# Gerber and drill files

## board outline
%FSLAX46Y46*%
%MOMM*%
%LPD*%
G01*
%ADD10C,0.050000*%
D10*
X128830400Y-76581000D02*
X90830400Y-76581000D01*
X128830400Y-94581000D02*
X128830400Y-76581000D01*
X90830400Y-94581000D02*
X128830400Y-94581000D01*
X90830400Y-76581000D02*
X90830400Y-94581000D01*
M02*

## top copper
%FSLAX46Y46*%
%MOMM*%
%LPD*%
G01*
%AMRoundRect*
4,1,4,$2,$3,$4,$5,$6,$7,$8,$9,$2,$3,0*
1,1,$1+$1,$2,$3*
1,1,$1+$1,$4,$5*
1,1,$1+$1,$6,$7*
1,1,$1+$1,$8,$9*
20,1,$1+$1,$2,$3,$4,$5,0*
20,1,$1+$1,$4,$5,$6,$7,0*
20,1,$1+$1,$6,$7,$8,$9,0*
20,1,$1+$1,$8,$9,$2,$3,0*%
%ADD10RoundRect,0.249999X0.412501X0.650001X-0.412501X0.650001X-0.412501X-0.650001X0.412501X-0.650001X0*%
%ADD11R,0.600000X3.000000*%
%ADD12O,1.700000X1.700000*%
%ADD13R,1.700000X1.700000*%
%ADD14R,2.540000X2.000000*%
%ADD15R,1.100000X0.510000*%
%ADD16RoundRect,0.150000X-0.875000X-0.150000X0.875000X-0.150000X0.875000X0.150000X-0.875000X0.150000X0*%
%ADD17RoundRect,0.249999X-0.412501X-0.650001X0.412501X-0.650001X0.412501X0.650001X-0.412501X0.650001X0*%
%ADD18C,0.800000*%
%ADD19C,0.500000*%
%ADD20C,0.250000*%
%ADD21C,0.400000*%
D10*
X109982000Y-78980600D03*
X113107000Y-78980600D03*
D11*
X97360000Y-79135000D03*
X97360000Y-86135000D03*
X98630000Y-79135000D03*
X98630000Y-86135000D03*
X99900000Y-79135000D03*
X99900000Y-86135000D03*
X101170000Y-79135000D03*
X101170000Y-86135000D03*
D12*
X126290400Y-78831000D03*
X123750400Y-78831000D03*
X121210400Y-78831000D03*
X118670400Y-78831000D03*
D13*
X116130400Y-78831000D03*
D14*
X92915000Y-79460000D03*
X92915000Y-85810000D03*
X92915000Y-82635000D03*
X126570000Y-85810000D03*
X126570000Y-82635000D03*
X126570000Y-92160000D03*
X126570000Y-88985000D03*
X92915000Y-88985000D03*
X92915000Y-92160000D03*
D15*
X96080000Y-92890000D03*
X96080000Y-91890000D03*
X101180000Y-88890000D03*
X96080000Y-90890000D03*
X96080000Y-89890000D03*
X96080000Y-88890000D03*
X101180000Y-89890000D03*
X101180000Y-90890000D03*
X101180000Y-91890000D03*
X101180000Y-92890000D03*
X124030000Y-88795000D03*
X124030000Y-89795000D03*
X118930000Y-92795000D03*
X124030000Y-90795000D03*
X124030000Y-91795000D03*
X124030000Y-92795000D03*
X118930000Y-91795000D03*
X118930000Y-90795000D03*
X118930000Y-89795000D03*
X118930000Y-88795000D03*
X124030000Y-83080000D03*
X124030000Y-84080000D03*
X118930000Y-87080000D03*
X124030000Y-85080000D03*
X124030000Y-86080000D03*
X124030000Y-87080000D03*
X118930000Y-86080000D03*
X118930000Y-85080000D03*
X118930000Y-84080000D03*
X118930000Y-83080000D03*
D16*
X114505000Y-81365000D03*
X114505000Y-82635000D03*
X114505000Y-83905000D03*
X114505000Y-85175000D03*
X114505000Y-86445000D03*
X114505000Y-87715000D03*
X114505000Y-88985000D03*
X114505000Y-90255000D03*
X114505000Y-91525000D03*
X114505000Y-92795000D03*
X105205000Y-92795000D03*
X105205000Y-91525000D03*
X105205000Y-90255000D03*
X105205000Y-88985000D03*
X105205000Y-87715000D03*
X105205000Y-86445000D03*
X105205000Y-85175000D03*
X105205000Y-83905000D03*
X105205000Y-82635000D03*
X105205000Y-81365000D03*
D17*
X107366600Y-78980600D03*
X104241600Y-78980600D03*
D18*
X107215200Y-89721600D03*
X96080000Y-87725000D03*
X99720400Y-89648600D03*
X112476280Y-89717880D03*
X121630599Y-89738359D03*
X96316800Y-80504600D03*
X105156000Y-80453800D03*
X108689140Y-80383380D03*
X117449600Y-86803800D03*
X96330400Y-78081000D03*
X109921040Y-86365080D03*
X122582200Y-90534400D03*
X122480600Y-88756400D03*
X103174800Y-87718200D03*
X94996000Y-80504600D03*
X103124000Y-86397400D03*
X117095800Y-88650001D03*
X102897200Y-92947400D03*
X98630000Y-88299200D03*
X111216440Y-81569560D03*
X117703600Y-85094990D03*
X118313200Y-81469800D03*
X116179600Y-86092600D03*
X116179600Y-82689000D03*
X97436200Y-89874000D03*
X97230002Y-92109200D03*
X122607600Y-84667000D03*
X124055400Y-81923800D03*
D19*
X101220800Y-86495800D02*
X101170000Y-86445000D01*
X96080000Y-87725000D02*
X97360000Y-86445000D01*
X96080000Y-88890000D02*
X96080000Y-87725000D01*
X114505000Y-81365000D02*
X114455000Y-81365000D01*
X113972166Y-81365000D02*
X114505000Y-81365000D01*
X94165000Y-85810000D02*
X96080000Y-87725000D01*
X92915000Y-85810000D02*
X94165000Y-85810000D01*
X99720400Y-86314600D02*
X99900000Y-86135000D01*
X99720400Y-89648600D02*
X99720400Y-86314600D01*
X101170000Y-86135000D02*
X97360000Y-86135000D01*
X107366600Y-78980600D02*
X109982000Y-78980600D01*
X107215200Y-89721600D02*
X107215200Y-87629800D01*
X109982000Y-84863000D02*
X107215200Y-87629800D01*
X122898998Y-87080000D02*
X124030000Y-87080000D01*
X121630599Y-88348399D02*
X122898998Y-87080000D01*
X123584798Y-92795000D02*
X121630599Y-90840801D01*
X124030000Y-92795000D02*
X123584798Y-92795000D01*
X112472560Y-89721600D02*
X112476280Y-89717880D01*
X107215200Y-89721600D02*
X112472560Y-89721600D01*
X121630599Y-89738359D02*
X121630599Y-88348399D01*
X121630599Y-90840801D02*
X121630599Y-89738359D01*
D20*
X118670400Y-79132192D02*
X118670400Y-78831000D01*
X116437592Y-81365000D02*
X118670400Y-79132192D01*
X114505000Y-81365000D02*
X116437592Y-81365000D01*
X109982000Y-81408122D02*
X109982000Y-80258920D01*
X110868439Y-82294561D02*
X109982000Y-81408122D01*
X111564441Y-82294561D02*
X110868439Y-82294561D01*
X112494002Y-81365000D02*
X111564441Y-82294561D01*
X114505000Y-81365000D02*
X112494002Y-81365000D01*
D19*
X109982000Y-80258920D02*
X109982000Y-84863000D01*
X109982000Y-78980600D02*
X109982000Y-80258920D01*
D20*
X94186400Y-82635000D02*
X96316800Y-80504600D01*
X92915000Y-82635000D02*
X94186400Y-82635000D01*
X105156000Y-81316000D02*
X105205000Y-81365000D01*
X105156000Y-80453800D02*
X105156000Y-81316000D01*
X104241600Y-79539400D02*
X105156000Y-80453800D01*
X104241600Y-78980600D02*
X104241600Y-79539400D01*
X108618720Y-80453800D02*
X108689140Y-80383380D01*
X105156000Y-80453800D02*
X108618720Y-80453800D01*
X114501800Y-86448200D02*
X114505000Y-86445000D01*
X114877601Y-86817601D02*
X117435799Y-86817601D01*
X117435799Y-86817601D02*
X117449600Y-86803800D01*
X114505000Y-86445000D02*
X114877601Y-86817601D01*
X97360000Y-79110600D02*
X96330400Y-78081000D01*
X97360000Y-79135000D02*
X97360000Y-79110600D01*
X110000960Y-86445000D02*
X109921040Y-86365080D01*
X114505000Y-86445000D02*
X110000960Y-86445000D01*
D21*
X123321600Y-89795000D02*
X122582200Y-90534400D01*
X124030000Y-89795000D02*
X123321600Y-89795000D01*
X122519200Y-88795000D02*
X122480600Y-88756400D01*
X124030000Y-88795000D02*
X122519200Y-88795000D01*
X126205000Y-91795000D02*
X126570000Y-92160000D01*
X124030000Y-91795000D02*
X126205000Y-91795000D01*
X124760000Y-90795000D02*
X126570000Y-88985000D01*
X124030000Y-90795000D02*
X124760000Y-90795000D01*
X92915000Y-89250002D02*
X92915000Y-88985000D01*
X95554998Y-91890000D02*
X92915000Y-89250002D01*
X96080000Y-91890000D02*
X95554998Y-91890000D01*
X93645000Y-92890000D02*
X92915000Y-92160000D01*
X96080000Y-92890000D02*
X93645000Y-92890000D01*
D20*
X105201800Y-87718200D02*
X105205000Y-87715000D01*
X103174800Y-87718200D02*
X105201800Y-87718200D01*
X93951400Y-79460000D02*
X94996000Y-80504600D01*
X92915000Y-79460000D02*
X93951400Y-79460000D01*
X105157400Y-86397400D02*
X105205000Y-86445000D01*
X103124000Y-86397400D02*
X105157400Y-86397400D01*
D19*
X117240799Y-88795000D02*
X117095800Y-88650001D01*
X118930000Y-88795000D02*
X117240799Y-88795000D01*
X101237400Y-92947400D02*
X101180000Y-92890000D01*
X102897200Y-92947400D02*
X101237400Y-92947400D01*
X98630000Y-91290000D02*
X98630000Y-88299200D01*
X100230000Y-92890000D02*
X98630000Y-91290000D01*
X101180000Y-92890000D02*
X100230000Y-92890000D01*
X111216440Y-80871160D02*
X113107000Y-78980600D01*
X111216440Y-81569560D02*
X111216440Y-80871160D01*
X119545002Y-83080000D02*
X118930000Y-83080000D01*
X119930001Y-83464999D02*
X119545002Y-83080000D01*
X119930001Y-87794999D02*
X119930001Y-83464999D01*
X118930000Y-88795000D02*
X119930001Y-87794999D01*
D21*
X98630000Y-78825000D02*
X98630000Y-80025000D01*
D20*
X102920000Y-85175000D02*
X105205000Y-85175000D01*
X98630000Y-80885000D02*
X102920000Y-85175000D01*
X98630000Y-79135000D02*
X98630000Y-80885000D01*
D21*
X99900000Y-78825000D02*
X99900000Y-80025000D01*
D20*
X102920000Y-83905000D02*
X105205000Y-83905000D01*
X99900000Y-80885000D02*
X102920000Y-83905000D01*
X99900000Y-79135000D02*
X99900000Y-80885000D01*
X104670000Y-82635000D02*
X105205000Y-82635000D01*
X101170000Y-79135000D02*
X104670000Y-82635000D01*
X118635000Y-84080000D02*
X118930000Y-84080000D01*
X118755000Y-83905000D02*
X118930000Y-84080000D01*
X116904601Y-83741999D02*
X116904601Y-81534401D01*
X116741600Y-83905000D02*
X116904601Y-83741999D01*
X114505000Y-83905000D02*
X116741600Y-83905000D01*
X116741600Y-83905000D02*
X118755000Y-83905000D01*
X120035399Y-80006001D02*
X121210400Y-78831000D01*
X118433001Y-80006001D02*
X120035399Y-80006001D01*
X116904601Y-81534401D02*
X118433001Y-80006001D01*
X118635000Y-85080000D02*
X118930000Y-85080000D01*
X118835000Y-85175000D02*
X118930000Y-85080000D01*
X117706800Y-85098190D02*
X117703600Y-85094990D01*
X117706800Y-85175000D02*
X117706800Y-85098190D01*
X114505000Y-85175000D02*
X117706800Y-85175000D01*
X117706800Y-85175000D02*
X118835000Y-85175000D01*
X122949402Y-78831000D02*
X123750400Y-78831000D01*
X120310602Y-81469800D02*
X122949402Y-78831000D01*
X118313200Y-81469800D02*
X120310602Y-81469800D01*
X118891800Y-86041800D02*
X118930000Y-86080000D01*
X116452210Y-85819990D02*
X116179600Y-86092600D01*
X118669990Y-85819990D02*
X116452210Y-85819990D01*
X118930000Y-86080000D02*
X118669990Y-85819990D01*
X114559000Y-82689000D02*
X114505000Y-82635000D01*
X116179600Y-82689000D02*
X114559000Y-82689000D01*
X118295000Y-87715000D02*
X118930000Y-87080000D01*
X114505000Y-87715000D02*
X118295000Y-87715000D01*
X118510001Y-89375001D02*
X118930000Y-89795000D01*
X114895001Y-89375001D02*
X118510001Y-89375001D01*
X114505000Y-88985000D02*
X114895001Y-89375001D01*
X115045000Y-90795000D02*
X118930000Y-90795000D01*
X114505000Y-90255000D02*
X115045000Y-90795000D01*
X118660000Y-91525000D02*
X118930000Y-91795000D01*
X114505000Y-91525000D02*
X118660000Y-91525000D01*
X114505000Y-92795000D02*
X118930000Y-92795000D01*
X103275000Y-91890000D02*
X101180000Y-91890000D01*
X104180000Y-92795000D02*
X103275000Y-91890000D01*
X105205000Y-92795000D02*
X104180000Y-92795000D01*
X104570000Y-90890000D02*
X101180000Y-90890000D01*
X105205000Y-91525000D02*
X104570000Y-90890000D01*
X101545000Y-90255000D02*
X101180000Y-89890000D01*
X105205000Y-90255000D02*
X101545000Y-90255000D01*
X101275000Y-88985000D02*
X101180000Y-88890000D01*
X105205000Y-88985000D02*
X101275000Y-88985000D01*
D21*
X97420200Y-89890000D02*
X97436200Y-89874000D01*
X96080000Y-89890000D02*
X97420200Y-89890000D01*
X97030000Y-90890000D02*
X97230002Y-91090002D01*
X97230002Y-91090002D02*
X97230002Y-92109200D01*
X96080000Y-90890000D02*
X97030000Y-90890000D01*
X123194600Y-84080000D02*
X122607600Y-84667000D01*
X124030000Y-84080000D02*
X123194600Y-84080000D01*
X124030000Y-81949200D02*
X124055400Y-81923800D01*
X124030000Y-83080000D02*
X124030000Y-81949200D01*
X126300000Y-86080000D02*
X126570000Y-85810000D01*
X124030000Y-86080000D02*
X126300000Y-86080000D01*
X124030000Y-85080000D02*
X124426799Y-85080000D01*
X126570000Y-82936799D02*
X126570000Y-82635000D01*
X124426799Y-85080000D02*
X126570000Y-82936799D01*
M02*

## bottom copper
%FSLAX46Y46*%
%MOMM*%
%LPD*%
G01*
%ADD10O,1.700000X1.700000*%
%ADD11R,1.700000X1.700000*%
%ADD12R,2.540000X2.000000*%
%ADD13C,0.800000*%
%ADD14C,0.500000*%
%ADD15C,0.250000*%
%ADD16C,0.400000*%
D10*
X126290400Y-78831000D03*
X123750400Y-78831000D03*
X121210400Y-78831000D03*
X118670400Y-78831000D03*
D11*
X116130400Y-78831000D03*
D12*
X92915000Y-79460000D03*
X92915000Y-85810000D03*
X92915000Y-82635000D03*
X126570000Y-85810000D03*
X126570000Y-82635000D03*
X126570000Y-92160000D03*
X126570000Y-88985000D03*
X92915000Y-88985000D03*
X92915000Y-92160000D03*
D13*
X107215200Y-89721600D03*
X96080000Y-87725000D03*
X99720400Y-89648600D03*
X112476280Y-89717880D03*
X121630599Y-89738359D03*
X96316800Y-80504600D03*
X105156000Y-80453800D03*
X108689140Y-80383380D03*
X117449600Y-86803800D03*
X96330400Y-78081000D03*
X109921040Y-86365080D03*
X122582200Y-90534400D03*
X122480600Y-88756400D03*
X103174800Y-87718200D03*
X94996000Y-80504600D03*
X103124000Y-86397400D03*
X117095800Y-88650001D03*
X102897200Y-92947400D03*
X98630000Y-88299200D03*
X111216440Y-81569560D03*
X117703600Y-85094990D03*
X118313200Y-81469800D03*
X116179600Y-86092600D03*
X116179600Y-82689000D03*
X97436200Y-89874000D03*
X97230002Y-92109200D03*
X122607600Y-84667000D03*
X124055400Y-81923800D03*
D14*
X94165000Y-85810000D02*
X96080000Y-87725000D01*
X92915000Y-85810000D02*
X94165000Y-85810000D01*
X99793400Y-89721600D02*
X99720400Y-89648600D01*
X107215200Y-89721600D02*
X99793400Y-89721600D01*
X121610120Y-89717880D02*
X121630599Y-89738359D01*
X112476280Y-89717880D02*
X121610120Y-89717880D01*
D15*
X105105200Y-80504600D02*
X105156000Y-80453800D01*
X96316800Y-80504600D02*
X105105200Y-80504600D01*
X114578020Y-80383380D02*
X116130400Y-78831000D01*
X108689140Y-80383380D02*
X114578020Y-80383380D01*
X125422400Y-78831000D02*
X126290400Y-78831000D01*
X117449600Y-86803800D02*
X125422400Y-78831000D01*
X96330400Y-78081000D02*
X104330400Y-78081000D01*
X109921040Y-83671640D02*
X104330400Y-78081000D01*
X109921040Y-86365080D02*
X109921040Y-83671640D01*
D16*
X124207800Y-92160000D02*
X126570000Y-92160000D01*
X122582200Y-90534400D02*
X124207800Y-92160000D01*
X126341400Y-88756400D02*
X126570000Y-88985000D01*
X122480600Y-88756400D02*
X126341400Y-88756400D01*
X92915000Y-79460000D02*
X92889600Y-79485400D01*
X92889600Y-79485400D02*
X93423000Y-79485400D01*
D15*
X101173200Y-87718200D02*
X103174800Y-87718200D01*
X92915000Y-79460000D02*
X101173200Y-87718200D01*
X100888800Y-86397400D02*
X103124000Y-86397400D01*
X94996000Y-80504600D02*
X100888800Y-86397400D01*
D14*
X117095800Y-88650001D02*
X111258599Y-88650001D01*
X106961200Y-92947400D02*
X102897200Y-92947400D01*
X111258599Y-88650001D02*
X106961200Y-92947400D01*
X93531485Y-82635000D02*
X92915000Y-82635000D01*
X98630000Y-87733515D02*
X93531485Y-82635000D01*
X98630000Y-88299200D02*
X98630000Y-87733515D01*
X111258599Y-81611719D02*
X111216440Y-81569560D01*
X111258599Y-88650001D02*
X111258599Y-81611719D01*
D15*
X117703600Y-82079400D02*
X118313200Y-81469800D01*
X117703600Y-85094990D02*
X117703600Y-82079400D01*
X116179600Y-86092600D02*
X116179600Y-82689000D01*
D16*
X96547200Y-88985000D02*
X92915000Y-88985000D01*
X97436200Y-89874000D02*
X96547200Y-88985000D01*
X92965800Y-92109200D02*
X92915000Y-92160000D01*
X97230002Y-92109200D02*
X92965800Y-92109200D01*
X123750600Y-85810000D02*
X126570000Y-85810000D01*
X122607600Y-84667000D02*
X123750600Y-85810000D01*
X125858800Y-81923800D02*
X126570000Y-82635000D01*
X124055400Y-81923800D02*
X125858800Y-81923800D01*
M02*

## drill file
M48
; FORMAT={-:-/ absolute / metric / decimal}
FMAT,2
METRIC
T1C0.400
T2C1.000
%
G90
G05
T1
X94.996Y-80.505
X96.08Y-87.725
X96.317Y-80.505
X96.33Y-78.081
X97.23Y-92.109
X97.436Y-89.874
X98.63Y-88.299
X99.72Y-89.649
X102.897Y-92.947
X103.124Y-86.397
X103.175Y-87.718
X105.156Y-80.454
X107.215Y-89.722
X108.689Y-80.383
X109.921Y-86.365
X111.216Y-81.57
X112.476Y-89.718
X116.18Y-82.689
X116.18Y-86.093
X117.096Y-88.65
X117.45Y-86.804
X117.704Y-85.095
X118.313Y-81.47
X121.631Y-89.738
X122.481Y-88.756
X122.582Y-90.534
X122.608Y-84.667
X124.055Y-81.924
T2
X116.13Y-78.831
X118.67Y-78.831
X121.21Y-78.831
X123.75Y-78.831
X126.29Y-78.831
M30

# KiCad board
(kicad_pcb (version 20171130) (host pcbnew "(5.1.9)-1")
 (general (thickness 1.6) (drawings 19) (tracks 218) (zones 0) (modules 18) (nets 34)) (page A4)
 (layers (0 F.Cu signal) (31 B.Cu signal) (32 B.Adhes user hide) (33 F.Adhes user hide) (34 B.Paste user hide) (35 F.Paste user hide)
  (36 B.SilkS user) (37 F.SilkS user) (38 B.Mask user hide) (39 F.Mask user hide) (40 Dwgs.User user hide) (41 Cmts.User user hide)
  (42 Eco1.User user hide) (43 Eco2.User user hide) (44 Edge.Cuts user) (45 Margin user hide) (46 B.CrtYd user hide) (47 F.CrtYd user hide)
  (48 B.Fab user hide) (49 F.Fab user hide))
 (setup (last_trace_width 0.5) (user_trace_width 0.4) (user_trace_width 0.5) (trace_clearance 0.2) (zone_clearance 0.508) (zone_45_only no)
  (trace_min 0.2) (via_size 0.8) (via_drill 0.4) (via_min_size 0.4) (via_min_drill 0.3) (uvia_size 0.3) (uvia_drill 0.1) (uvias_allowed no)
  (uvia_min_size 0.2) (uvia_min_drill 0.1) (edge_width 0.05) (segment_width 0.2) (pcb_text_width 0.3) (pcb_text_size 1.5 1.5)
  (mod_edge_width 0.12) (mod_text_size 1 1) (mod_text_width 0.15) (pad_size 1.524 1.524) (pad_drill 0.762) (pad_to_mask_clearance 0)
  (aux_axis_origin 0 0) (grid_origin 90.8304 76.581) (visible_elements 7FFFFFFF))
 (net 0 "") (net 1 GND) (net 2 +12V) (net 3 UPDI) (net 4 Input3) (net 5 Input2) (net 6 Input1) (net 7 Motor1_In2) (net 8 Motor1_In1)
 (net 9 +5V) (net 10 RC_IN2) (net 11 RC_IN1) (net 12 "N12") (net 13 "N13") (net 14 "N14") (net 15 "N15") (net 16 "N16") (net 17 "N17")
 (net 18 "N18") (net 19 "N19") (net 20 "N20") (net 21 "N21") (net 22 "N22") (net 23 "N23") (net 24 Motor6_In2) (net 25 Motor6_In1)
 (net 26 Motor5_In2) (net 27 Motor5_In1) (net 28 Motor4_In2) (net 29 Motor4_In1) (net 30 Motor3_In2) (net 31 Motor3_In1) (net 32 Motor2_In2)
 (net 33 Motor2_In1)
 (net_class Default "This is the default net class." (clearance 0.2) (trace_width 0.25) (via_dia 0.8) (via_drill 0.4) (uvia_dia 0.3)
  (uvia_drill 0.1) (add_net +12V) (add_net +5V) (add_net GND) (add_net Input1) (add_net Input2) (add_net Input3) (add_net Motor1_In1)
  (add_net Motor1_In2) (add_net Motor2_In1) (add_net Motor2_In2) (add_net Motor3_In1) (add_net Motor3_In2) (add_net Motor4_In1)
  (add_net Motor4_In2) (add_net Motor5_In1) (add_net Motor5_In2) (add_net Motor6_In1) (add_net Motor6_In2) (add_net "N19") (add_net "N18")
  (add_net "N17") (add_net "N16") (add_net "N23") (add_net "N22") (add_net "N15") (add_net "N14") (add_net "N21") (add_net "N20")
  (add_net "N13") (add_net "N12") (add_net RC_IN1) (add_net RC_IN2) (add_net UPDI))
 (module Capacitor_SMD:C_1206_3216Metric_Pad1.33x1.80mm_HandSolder (layer F.Cu) (at 111.5445 78.9806 180)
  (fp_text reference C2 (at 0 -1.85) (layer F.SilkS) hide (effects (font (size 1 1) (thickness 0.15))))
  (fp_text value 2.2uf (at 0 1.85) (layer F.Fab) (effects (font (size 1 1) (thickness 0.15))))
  (pad 2 smd roundrect (at 1.5625 0 180) (size 1.325 1.8) (layers F.Cu F.Paste F.Mask) (roundrect_rratio 0.1886784905660377) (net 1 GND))
  (pad 1 smd roundrect (at -1.5625 0 180) (size 1.325 1.8) (layers F.Cu F.Paste F.Mask) (roundrect_rratio 0.1886784905660377) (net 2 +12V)))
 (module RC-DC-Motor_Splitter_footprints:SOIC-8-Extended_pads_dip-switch (layer F.Cu) (at 99.265 82.635 180)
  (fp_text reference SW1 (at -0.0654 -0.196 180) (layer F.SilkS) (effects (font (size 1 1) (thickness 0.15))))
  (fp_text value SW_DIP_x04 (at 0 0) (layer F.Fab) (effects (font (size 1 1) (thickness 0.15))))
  (pad 4 smd rect (at 1.905 3.5 180) (size 0.6 3) (layers F.Cu F.Paste F.Mask) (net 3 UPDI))
  (pad 5 smd rect (at 1.905 -3.5 180) (size 0.6 3) (layers F.Cu F.Paste F.Mask) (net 1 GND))
  (pad 3 smd rect (at 0.635 3.5 180) (size 0.6 3) (layers F.Cu F.Paste F.Mask) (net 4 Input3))
  (pad 6 smd rect (at 0.635 -3.5 180) (size 0.6 3) (layers F.Cu F.Paste F.Mask) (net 1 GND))
  (pad 2 smd rect (at -0.635 3.5 180) (size 0.6 3) (layers F.Cu F.Paste F.Mask) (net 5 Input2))
  (pad 7 smd rect (at -0.635 -3.5 180) (size 0.6 3) (layers F.Cu F.Paste F.Mask) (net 1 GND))
  (pad 1 smd rect (at -1.905 3.5 180) (size 0.6 3) (layers F.Cu F.Paste F.Mask) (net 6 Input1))
  (pad 8 smd rect (at -1.905 -3.5 180) (size 0.6 3) (layers F.Cu F.Paste F.Mask) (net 1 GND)))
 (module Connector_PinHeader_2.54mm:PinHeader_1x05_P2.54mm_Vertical (layer F.Cu) (at 116.1304 78.831 90)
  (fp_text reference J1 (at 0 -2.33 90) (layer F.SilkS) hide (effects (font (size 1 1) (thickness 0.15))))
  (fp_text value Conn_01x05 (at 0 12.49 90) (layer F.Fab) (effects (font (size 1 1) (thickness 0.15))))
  (pad 5 thru_hole oval (at 0 10.16 90) (size 1.7 1.7) (drill 1) (layers *.Cu *.Mask) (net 3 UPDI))
  (pad 4 thru_hole oval (at 0 7.62 90) (size 1.7 1.7) (drill 1) (layers *.Cu *.Mask) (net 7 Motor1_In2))
  (pad 3 thru_hole oval (at 0 5.08 90) (size 1.7 1.7) (drill 1) (layers *.Cu *.Mask) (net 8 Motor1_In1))
  (pad 2 thru_hole oval (at 0 2.54 90) (size 1.7 1.7) (drill 1) (layers *.Cu *.Mask) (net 1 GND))
  (pad 1 thru_hole rect (at 0 0 90) (size 1.7 1.7) (drill 1) (layers *.Cu *.Mask) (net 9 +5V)))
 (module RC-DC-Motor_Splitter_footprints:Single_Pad (layer F.Cu) (at 92.915 79.46 90)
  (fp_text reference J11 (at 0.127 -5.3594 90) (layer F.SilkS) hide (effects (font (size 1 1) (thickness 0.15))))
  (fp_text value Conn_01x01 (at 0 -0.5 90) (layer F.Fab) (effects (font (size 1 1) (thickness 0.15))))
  (pad 1 smd rect (at 0 0 90) (size 2 2.54) (layers F.Cu F.Paste F.Mask) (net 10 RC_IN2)))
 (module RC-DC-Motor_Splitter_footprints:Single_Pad (layer B.Cu) (at 92.915 79.46 270)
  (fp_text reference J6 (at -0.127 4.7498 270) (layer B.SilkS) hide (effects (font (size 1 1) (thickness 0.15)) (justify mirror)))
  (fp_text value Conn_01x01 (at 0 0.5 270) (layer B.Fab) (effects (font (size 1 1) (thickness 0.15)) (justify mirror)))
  (pad 1 smd rect (at 0 0 270) (size 2 2.54) (layers B.Cu B.Paste B.Mask) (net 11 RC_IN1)))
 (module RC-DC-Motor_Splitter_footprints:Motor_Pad (layer F.Cu) (at 92.915 82.635 270)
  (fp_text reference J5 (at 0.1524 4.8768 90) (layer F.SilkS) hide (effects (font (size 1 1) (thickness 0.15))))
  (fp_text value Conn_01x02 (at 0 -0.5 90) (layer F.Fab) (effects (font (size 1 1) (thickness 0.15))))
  (pad 2 smd rect (at 3.175 0 270) (size 2 2.54) (layers F.Cu F.Paste F.Mask) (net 1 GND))
  (pad 1 smd rect (at 0 0 270) (size 2 2.54) (layers F.Cu F.Paste F.Mask) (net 9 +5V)))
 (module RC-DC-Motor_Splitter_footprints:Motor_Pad (layer B.Cu) (at 92.915 82.635 270)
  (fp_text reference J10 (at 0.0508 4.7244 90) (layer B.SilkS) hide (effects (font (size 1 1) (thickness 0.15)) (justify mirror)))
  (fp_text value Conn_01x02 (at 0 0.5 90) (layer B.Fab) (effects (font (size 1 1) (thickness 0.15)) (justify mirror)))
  (pad 2 smd rect (at 3.175 0 270) (size 2 2.54) (layers B.Cu B.Paste B.Mask) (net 1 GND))
  (pad 1 smd rect (at 0 0 270) (size 2 2.54) (layers B.Cu B.Paste B.Mask) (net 2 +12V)))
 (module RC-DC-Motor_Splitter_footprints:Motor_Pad (layer F.Cu) (at 126.57 82.635 270)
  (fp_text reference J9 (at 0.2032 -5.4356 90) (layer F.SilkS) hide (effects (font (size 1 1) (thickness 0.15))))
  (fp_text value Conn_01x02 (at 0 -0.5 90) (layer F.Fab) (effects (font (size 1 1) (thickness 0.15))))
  (pad 2 smd rect (at 3.175 0 270) (size 2 2.54) (layers F.Cu F.Paste F.Mask) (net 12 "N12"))
  (pad 1 smd rect (at 0 0 270) (size 2 2.54) (layers F.Cu F.Paste F.Mask) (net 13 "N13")))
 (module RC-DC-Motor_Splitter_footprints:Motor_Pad (layer B.Cu) (at 126.57 82.635 270)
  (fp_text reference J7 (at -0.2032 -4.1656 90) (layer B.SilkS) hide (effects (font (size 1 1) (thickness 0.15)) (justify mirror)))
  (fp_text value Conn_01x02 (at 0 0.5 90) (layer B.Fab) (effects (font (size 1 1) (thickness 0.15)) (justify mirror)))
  (pad 2 smd rect (at 3.175 0 270) (size 2 2.54) (layers B.Cu B.Paste B.Mask) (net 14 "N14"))
  (pad 1 smd rect (at 0 0 270) (size 2 2.54) (layers B.Cu B.Paste B.Mask) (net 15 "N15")))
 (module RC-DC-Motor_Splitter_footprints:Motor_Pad (layer F.Cu) (at 126.57 88.985 270)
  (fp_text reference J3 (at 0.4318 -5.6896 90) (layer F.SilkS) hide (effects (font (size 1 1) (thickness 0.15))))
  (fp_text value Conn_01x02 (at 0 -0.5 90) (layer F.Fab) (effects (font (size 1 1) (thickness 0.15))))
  (pad 2 smd rect (at 3.175 0 270) (size 2 2.54) (layers F.Cu F.Paste F.Mask) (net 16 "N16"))
  (pad 1 smd rect (at 0 0 270) (size 2 2.54) (layers F.Cu F.Paste F.Mask) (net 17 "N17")))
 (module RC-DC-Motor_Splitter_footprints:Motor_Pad (layer B.Cu) (at 126.57 88.985 270)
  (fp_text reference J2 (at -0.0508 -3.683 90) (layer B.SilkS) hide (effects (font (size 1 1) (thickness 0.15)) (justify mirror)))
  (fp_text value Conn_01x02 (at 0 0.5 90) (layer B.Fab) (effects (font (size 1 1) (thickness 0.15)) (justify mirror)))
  (pad 2 smd rect (at 3.175 0 270) (size 2 2.54) (layers B.Cu B.Paste B.Mask) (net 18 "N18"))
  (pad 1 smd rect (at 0 0 270) (size 2 2.54) (layers B.Cu B.Paste B.Mask) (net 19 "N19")))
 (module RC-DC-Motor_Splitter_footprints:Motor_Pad (layer B.Cu) (at 92.915 92.16 90)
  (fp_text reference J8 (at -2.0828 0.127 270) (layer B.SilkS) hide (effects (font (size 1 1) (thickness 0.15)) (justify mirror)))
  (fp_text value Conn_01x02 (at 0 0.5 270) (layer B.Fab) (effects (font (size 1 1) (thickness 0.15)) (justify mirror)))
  (pad 2 smd rect (at 3.175 0 90) (size 2 2.54) (layers B.Cu B.Paste B.Mask) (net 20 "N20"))
  (pad 1 smd rect (at 0 0 90) (size 2 2.54) (layers B.Cu B.Paste B.Mask) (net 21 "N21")))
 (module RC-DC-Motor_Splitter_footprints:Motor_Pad (layer F.Cu) (at 92.915 92.16 90)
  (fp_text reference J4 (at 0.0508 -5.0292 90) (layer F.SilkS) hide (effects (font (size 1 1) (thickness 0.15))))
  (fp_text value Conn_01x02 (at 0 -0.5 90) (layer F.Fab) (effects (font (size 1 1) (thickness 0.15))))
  (pad 2 smd rect (at 3.175 0 90) (size 2 2.54) (layers F.Cu F.Paste F.Mask) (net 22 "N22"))
  (pad 1 smd rect (at 0 0 90) (size 2 2.54) (layers F.Cu F.Paste F.Mask) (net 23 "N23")))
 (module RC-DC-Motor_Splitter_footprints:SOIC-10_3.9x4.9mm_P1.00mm (layer F.Cu) (at 98.63 90.89 180)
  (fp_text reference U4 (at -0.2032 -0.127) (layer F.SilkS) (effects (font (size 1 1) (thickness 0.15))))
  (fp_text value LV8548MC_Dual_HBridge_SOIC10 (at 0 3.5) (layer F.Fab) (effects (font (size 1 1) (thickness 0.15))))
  (pad 10 smd rect (at 2.55 -2 180) (size 1.1 0.51) (layers F.Cu F.Paste F.Mask) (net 23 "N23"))
  (pad 9 smd rect (at 2.55 -1 180) (size 1.1 0.51) (layers F.Cu F.Paste F.Mask) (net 22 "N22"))
  (pad 5 smd rect (at -2.55 2 180) (size 1.1 0.51) (layers F.Cu F.Paste F.Mask) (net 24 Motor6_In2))
  (pad 8 smd rect (at 2.55 0 180) (size 1.1 0.51) (layers F.Cu F.Paste F.Mask) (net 21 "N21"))
  (pad 7 smd rect (at 2.55 1 180) (size 1.1 0.51) (layers F.Cu F.Paste F.Mask) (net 20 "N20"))
  (pad 6 smd rect (at 2.55 2 180) (size 1.1 0.51) (layers F.Cu F.Paste F.Mask) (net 1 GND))
  (pad 4 smd rect (at -2.55 1 180) (size 1.1 0.51) (layers F.Cu F.Paste F.Mask) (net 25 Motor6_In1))
  (pad 3 smd rect (at -2.55 0 180) (size 1.1 0.51) (layers F.Cu F.Paste F.Mask) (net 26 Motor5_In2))
  (pad 2 smd rect (at -2.55 -1 180) (size 1.1 0.51) (layers F.Cu F.Paste F.Mask) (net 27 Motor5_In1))
  (pad 1 smd rect (at -2.55 -2 180) (size 1.1 0.51) (layers F.Cu F.Paste F.Mask) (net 2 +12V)))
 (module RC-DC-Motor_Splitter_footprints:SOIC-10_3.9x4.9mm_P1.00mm (layer F.Cu) (at 121.48 90.795)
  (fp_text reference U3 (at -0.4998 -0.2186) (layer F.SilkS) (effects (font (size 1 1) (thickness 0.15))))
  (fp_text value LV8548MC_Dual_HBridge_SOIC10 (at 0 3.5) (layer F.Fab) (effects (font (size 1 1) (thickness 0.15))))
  (pad 10 smd rect (at 2.55 -2) (size 1.1 0.51) (layers F.Cu F.Paste F.Mask) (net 19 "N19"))
  (pad 9 smd rect (at 2.55 -1) (size 1.1 0.51) (layers F.Cu F.Paste F.Mask) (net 18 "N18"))
  (pad 5 smd rect (at -2.55 2) (size 1.1 0.51) (layers F.Cu F.Paste F.Mask) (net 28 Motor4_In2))
  (pad 8 smd rect (at 2.55 0) (size 1.1 0.51) (layers F.Cu F.Paste F.Mask) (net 17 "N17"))
  (pad 7 smd rect (at 2.55 1) (size 1.1 0.51) (layers F.Cu F.Paste F.Mask) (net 16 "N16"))
  (pad 6 smd rect (at 2.55 2) (size 1.1 0.51) (layers F.Cu F.Paste F.Mask) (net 1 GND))
  (pad 4 smd rect (at -2.55 1) (size 1.1 0.51) (layers F.Cu F.Paste F.Mask) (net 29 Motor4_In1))
  (pad 3 smd rect (at -2.55 0) (size 1.1 0.51) (layers F.Cu F.Paste F.Mask) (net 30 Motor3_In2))
  (pad 2 smd rect (at -2.55 -1) (size 1.1 0.51) (layers F.Cu F.Paste F.Mask) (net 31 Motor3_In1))
  (pad 1 smd rect (at -2.55 -2) (size 1.1 0.51) (layers F.Cu F.Paste F.Mask) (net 2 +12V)))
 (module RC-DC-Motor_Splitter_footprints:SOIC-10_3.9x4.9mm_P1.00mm (layer F.Cu) (at 121.48 85.08)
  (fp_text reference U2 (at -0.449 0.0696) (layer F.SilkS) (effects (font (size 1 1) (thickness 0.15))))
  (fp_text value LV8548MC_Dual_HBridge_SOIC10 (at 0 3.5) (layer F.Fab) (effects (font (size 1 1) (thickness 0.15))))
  (pad 10 smd rect (at 2.55 -2) (size 1.1 0.51) (layers F.Cu F.Paste F.Mask) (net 15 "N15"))
  (pad 9 smd rect (at 2.55 -1) (size 1.1 0.51) (layers F.Cu F.Paste F.Mask) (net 14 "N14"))
  (pad 5 smd rect (at -2.55 2) (size 1.1 0.51) (layers F.Cu F.Paste F.Mask) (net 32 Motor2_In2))
  (pad 8 smd rect (at 2.55 0) (size 1.1 0.51) (layers F.Cu F.Paste F.Mask) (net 13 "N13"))
  (pad 7 smd rect (at 2.55 1) (size 1.1 0.51) (layers F.Cu F.Paste F.Mask) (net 12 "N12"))
  (pad 6 smd rect (at 2.55 2) (size 1.1 0.51) (layers F.Cu F.Paste F.Mask) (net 1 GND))
  (pad 4 smd rect (at -2.55 1) (size 1.1 0.51) (layers F.Cu F.Paste F.Mask) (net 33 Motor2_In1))
  (pad 3 smd rect (at -2.55 0) (size 1.1 0.51) (layers F.Cu F.Paste F.Mask) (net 7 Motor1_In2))
  (pad 2 smd rect (at -2.55 -1) (size 1.1 0.51) (layers F.Cu F.Paste F.Mask) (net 8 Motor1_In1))
  (pad 1 smd rect (at -2.55 -2) (size 1.1 0.51) (layers F.Cu F.Paste F.Mask) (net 2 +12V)))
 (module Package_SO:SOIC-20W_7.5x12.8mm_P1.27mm (layer F.Cu) (at 109.855 87.08)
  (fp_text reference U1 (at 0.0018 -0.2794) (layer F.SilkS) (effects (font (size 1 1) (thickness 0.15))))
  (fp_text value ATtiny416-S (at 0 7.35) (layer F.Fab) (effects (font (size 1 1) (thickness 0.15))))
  (pad 20 smd roundrect (at 4.65 -5.715) (size 2.05 0.6) (layers F.Cu F.Paste F.Mask) (roundrect_rratio 0.25) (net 1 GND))
  (pad 19 smd roundrect (at 4.65 -4.445) (size 2.05 0.6) (layers F.Cu F.Paste F.Mask) (roundrect_rratio 0.25) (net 33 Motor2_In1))
  (pad 18 smd roundrect (at 4.65 -3.175) (size 2.05 0.6) (layers F.Cu F.Paste F.Mask) (roundrect_rratio 0.25) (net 8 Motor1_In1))
  (pad 17 smd roundrect (at 4.65 -1.905) (size 2.05 0.6) (layers F.Cu F.Paste F.Mask) (roundrect_rratio 0.25) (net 7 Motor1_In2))
  (pad 16 smd roundrect (at 4.65 -0.635) (size 2.05 0.6) (layers F.Cu F.Paste F.Mask) (roundrect_rratio 0.25) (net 3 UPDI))
  (pad 15 smd roundrect (at 4.65 0.635) (size 2.05 0.6) (layers F.Cu F.Paste F.Mask) (roundrect_rratio 0.25) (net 32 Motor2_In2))
  (pad 14 smd roundrect (at 4.65 1.905) (size 2.05 0.6) (layers F.Cu F.Paste F.Mask) (roundrect_rratio 0.25) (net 31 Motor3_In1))
  (pad 13 smd roundrect (at 4.65 3.175) (size 2.05 0.6) (layers F.Cu F.Paste F.Mask) (roundrect_rratio 0.25) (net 30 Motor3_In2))
  (pad 12 smd roundrect (at 4.65 4.445) (size 2.05 0.6) (layers F.Cu F.Paste F.Mask) (roundrect_rratio 0.25) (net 29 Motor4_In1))
  (pad 11 smd roundrect (at 4.65 5.715) (size 2.05 0.6) (layers F.Cu F.Paste F.Mask) (roundrect_rratio 0.25) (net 28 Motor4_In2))
  (pad 10 smd roundrect (at -4.65 5.715) (size 2.05 0.6) (layers F.Cu F.Paste F.Mask) (roundrect_rratio 0.25) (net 27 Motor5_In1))
  (pad 9 smd roundrect (at -4.65 4.445) (size 2.05 0.6) (layers F.Cu F.Paste F.Mask) (roundrect_rratio 0.25) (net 26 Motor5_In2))
  (pad 8 smd roundrect (at -4.65 3.175) (size 2.05 0.6) (layers F.Cu F.Paste F.Mask) (roundrect_rratio 0.25) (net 25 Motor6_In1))
  (pad 7 smd roundrect (at -4.65 1.905) (size 2.05 0.6) (layers F.Cu F.Paste F.Mask) (roundrect_rratio 0.25) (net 24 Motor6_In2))
  (pad 6 smd roundrect (at -4.65 0.635) (size 2.05 0.6) (layers F.Cu F.Paste F.Mask) (roundrect_rratio 0.25) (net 11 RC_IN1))
  (pad 5 smd roundrect (at -4.65 -0.635) (size 2.05 0.6) (layers F.Cu F.Paste F.Mask) (roundrect_rratio 0.25) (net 10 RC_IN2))
  (pad 4 smd roundrect (at -4.65 -1.905) (size 2.05 0.6) (layers F.Cu F.Paste F.Mask) (roundrect_rratio 0.25) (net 4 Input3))
  (pad 3 smd roundrect (at -4.65 -3.175) (size 2.05 0.6) (layers F.Cu F.Paste F.Mask) (roundrect_rratio 0.25) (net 5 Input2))
  (pad 2 smd roundrect (at -4.65 -4.445) (size 2.05 0.6) (layers F.Cu F.Paste F.Mask) (roundrect_rratio 0.25) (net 6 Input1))
  (pad 1 smd roundrect (at -4.65 -5.715) (size 2.05 0.6) (layers F.Cu F.Paste F.Mask) (roundrect_rratio 0.25) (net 9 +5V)))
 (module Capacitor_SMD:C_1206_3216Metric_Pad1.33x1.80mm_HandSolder (layer F.Cu) (at 105.8041 78.9806)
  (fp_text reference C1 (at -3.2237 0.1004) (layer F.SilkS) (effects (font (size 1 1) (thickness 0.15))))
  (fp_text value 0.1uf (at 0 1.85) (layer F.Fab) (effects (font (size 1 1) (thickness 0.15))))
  (pad 2 smd roundrect (at 1.5625 0) (size 1.325 1.8) (layers F.Cu F.Paste F.Mask) (roundrect_rratio 0.1886784905660377) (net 1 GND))
  (pad 1 smd roundrect (at -1.5625 0) (size 1.325 1.8) (layers F.Cu F.Paste F.Mask) (roundrect_rratio 0.1886784905660377) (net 9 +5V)))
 (gr_line (start 128.8304 76.581) (end 90.8304 76.581) (layer Edge.Cuts) (width 0.05))
 (gr_line (start 128.8304 94.581) (end 128.8304 76.581) (layer Edge.Cuts) (width 0.05))
 (gr_line (start 90.8304 94.581) (end 128.8304 94.581) (layer Edge.Cuts) (width 0.05))
 (gr_line (start 90.8304 76.581) (end 90.8304 94.581) (layer Edge.Cuts) (width 0.05))
 (via (at 107.2152 89.7216) (size 0.8) (drill 0.4) (layers F.Cu B.Cu) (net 1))
 (segment (start 101.2208 86.4958) (end 101.17 86.445) (width 0.5) (layer F.Cu) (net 1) (status 30))
 (segment (start 96.08 87.725) (end 97.36 86.445) (width 0.5) (layer F.Cu) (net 1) (status 20))
 (segment (start 96.08 88.89) (end 96.08 87.725) (width 0.5) (layer F.Cu) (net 1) (status 10))
 (segment (start 114.505 81.365) (end 114.455 81.365) (width 0.5) (layer F.Cu) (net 1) (status 30))
 (segment (start 113.972166 81.365) (end 114.505 81.365) (width 0.5) (layer F.Cu) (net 1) (status 30))
 (via (at 96.08 87.725) (size 0.8) (drill 0.4) (layers F.Cu B.Cu) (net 1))
 (segment (start 94.165 85.81) (end 96.08 87.725) (width 0.5) (layer B.Cu) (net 1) (status 10))
 (segment (start 92.915 85.81) (end 94.165 85.81) (width 0.5) (layer B.Cu) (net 1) (status 30))
 (segment (start 94.165 85.81) (end 96.08 87.725) (width 0.5) (layer F.Cu) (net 1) (status 10))
 (segment (start 92.915 85.81) (end 94.165 85.81) (width 0.5) (layer F.Cu) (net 1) (status 30))
 (via (at 99.7204 89.6486) (size 0.8) (drill 0.4) (layers F.Cu B.Cu) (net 1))
 (segment (start 99.7934 89.7216) (end 99.7204 89.6486) (width 0.5) (layer B.Cu) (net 1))
 (segment (start 107.2152 89.7216) (end 99.7934 89.7216) (width 0.5) (layer B.Cu) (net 1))
 (segment (start 99.7204 86.3146) (end 99.9 86.135) (width 0.5) (layer F.Cu) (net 1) (status 30))
 (segment (start 99.7204 89.6486) (end 99.7204 86.3146) (width 0.5) (layer F.Cu) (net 1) (status 20))
 (segment (start 101.17 86.135) (end 97.36 86.135) (width 0.5) (layer F.Cu) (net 1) (status 30))
 (segment (start 107.3666 78.9806) (end 109.982 78.9806) (width 0.5) (layer F.Cu) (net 1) (status 30))
 (segment (start 107.2152 89.7216) (end 107.2152 87.6298) (width 0.5) (layer F.Cu) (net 1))
 (segment (start 109.982 84.863) (end 107.2152 87.6298) (width 0.5) (layer F.Cu) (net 1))
 (segment (start 122.898998 87.08) (end 124.03 87.08) (width 0.5) (layer F.Cu) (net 1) (status 20))
 (segment (start 121.630599 88.348399) (end 122.898998 87.08) (width 0.5) (layer F.Cu) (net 1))
 (segment (start 123.584798 92.795) (end 121.630599 90.840801) (width 0.5) (layer F.Cu) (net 1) (status 10))
 (segment (start 124.03 92.795) (end 123.584798 92.795) (width 0.5) (layer F.Cu) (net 1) (status 30))
 (via (at 112.47628 89.71788) (size 0.8) (drill 0.4) (layers F.Cu B.Cu) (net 1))
 (segment (start 112.47256 89.7216) (end 112.47628 89.71788) (width 0.5) (layer F.Cu) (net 1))
 (segment (start 107.2152 89.7216) (end 112.47256 89.7216) (width 0.5) (layer F.Cu) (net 1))
 (via (at 121.630599 89.738359) (size 0.8) (drill 0.4) (layers F.Cu B.Cu) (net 1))
 (segment (start 121.61012 89.71788) (end 121.630599 89.738359) (width 0.5) (layer B.Cu) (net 1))
 (segment (start 112.47628 89.71788) (end 121.61012 89.71788) (width 0.5) (layer B.Cu) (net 1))
 (segment (start 121.630599 89.738359) (end 121.630599 88.348399) (width 0.5) (layer F.Cu) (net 1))
 (segment (start 121.630599 90.840801) (end 121.630599 89.738359) (width 0.5) (layer F.Cu) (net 1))
 (segment (start 118.6704 79.132192) (end 118.6704 78.831) (width 0.25) (layer F.Cu) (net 1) (status 30))
 (segment (start 116.437592 81.365) (end 118.6704 79.132192) (width 0.25) (layer F.Cu) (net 1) (status 20))
 (segment (start 114.505 81.365) (end 116.437592 81.365) (width 0.25) (layer F.Cu) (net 1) (status 10))
 (segment (start 109.982 81.408122) (end 109.982 80.25892) (width 0.25) (layer F.Cu) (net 1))
 (segment (start 110.868439 82.294561) (end 109.982 81.408122) (width 0.25) (layer F.Cu) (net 1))
 (segment (start 111.564441 82.294561) (end 110.868439 82.294561) (width 0.25) (layer F.Cu) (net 1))
 (segment (start 112.494002 81.365) (end 111.564441 82.294561) (width 0.25) (layer F.Cu) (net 1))
 (segment (start 114.505 81.365) (end 112.494002 81.365) (width 0.25) (layer F.Cu) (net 1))
 (segment (start 109.982 80.25892) (end 109.982 84.863) (width 0.5) (layer F.Cu) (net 1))
 (segment (start 109.982 78.9806) (end 109.982 80.25892) (width 0.5) (layer F.Cu) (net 1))
 (via (at 96.3168 80.5046) (size 0.8) (drill 0.4) (layers F.Cu B.Cu) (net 9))
 (segment (start 94.1864 82.635) (end 96.3168 80.5046) (width 0.25) (layer F.Cu) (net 9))
 (segment (start 92.915 82.635) (end 94.1864 82.635) (width 0.25) (layer F.Cu) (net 9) (status 10))
 (via (at 105.156 80.4538) (size 0.8) (drill 0.4) (layers F.Cu B.Cu) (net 9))
 (segment (start 105.1052 80.5046) (end 105.156 80.4538) (width 0.25) (layer B.Cu) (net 9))
 (segment (start 96.3168 80.5046) (end 105.1052 80.5046) (width 0.25) (layer B.Cu) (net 9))
 (segment (start 105.156 81.316) (end 105.205 81.365) (width 0.25) (layer F.Cu) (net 9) (status 30))
 (segment (start 105.156 80.4538) (end 105.156 81.316) (width 0.25) (layer F.Cu) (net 9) (status 20))
 (segment (start 104.2416 79.5394) (end 105.156 80.4538) (width 0.25) (layer F.Cu) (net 9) (status 10))
 (segment (start 104.2416 78.9806) (end 104.2416 79.5394) (width 0.25) (layer F.Cu) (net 9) (status 30))
 (via (at 108.68914 80.38338) (size 0.8) (drill 0.4) (layers F.Cu B.Cu) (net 9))
 (segment (start 108.61872 80.4538) (end 108.68914 80.38338) (width 0.25) (layer F.Cu) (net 9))
 (segment (start 105.156 80.4538) (end 108.61872 80.4538) (width 0.25) (layer F.Cu) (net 9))
 (segment (start 114.57802 80.38338) (end 116.1304 78.831) (width 0.25) (layer B.Cu) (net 9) (status 20))
 (segment (start 108.68914 80.38338) (end 114.57802 80.38338) (width 0.25) (layer B.Cu) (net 9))
 (segment (start 114.5018 86.4482) (end 114.505 86.445) (width 0.25) (layer F.Cu) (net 3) (status 30))
 (via (at 117.4496 86.8038) (size 0.8) (drill 0.4) (layers F.Cu B.Cu) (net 3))
 (segment (start 114.877601 86.817601) (end 117.435799 86.817601) (width 0.25) (layer F.Cu) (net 3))
 (segment (start 117.435799 86.817601) (end 117.4496 86.8038) (width 0.25) (layer F.Cu) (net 3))
 (segment (start 114.505 86.445) (end 114.877601 86.817601) (width 0.25) (layer F.Cu) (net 3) (status 10))
 (segment (start 125.4224 78.831) (end 126.2904 78.831) (width 0.25) (layer B.Cu) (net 3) (status 20))
 (segment (start 117.4496 86.8038) (end 125.4224 78.831) (width 0.25) (layer B.Cu) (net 3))
 (via (at 96.3304 78.081) (size 0.8) (drill 0.4) (layers F.Cu B.Cu) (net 3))
 (segment (start 97.36 79.1106) (end 96.3304 78.081) (width 0.25) (layer F.Cu) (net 3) (status 10))
 (segment (start 97.36 79.135) (end 97.36 79.1106) (width 0.25) (layer F.Cu) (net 3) (status 30))
 (segment (start 96.3304 78.081) (end 104.3304 78.081) (width 0.25) (layer B.Cu) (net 3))
 (via (at 109.92104 86.36508) (size 0.8) (drill 0.4) (layers F.Cu B.Cu) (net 3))
 (segment (start 110.00096 86.445) (end 109.92104 86.36508) (width 0.25) (layer F.Cu) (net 3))
 (segment (start 114.505 86.445) (end 110.00096 86.445) (width 0.25) (layer F.Cu) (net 3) (status 10))
 (segment (start 109.92104 83.67164) (end 104.3304 78.081) (width 0.25) (layer B.Cu) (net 3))
 (segment (start 109.92104 86.36508) (end 109.92104 83.67164) (width 0.25) (layer B.Cu) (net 3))
 (segment (start 123.3216 89.795) (end 122.5822 90.5344) (width 0.4) (layer F.Cu) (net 18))
 (via (at 122.5822 90.5344) (size 0.8) (drill 0.4) (layers F.Cu B.Cu) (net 18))
 (segment (start 124.03 89.795) (end 123.3216 89.795) (width 0.4) (layer F.Cu) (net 18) (status 10))
 (segment (start 124.2078 92.16) (end 126.57 92.16) (width 0.4) (layer B.Cu) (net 18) (status 20))
 (segment (start 122.5822 90.5344) (end 124.2078 92.16) (width 0.4) (layer B.Cu) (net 18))
 (via (at 122.4806 88.7564) (size 0.8) (drill 0.4) (layers F.Cu B.Cu) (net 19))
 (segment (start 122.5192 88.795) (end 122.4806 88.7564) (width 0.4) (layer F.Cu) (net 19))
 (segment (start 124.03 88.795) (end 122.5192 88.795) (width 0.4) (layer F.Cu) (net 19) (status 10))
 (segment (start 126.3414 88.7564) (end 126.57 88.985) (width 0.4) (layer B.Cu) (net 19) (status 30))
 (segment (start 122.4806 88.7564) (end 126.3414 88.7564) (width 0.4) (layer B.Cu) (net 19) (status 20))
 (segment (start 126.205 91.795) (end 126.57 92.16) (width 0.4) (layer F.Cu) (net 16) (status 30))
 (segment (start 124.03 91.795) (end 126.205 91.795) (width 0.4) (layer F.Cu) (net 16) (status 30))
 (segment (start 124.76 90.795) (end 126.57 88.985) (width 0.4) (layer F.Cu) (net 17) (status 20))
 (segment (start 124.03 90.795) (end 124.76 90.795) (width 0.4) (layer F.Cu) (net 17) (status 10))
 (segment (start 92.915 89.250002) (end 92.915 88.985) (width 0.4) (layer F.Cu) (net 22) (status 30))
 (segment (start 95.554998 91.89) (end 92.915 89.250002) (width 0.4) (layer F.Cu) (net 22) (status 30))
 (segment (start 96.08 91.89) (end 95.554998 91.89) (width 0.4) (layer F.Cu) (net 22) (status 30))
 (segment (start 93.645 92.89) (end 92.915 92.16) (width 0.4) (layer F.Cu) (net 23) (status 30))
 (segment (start 96.08 92.89) (end 93.645 92.89) (width 0.4) (layer F.Cu) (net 23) (status 30))
 (segment (start 92.915 79.46) (end 92.8896 79.4854) (width 0.4) (layer B.Cu) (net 11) (status 30))
 (segment (start 92.8896 79.4854) (end 93.423 79.4854) (width 0.4) (layer B.Cu) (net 11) (status 30))
 (via (at 103.1748 87.7182) (size 0.8) (drill 0.4) (layers F.Cu B.Cu) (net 11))
 (segment (start 101.1732 87.7182) (end 103.1748 87.7182) (width 0.25) (layer B.Cu) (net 11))
 (segment (start 92.915 79.46) (end 101.1732 87.7182) (width 0.25) (layer B.Cu) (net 11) (status 10))
 (segment (start 105.2018 87.7182) (end 105.205 87.715) (width 0.25) (layer F.Cu) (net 11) (status 30))
 (segment (start 103.1748 87.7182) (end 105.2018 87.7182) (width 0.25) (layer F.Cu) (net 11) (status 20))
 (via (at 94.996 80.5046) (size 0.8) (drill 0.4) (layers F.Cu B.Cu) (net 10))
 (segment (start 93.9514 79.46) (end 94.996 80.5046) (width 0.25) (layer F.Cu) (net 10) (status 10))
 (segment (start 92.915 79.46) (end 93.9514 79.46) (width 0.25) (layer F.Cu) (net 10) (status 30))
 (via (at 103.124 86.3974) (size 0.8) (drill 0.4) (layers F.Cu B.Cu) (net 10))
 (segment (start 100.8888 86.3974) (end 103.124 86.3974) (width 0.25) (layer B.Cu) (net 10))
 (segment (start 94.996 80.5046) (end 100.8888 86.3974) (width 0.25) (layer B.Cu) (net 10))
 (segment (start 105.1574 86.3974) (end 105.205 86.445) (width 0.25) (layer F.Cu) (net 10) (status 30))
 (segment (start 103.124 86.3974) (end 105.1574 86.3974) (width 0.25) (layer F.Cu) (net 10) (status 20))
 (via (at 117.0958 88.650001) (size 0.8) (drill 0.4) (layers F.Cu B.Cu) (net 2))
 (segment (start 117.240799 88.795) (end 117.0958 88.650001) (width 0.5) (layer F.Cu) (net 2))
 (segment (start 118.93 88.795) (end 117.240799 88.795) (width 0.5) (layer F.Cu) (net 2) (status 10))
 (via (at 102.8972 92.9474) (size 0.8) (drill 0.4) (layers F.Cu B.Cu) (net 2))
 (segment (start 101.2374 92.9474) (end 101.18 92.89) (width 0.5) (layer F.Cu) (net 2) (status 30))
 (segment (start 102.8972 92.9474) (end 101.2374 92.9474) (width 0.5) (layer F.Cu) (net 2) (status 20))
 (segment (start 117.0958 88.650001) (end 111.258599 88.650001) (width 0.5) (layer B.Cu) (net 2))
 (segment (start 106.9612 92.9474) (end 102.8972 92.9474) (width 0.5) (layer B.Cu) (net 2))
 (segment (start 111.258599 88.650001) (end 106.9612 92.9474) (width 0.5) (layer B.Cu) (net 2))
 (via (at 98.63 88.2992) (size 0.8) (drill 0.4) (layers F.Cu B.Cu) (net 2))
 (segment (start 98.63 91.29) (end 98.63 88.2992) (width 0.5) (layer F.Cu) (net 2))
 (segment (start 100.23 92.89) (end 98.63 91.29) (width 0.5) (layer F.Cu) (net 2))
 (segment (start 101.18 92.89) (end 100.23 92.89) (width 0.5) (layer F.Cu) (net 2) (status 10))
 (segment (start 93.531485 82.635) (end 92.915 82.635) (width 0.5) (layer B.Cu) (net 2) (status 30))
 (segment (start 98.63 87.733515) (end 93.531485 82.635) (width 0.5) (layer B.Cu) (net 2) (status 20))
 (segment (start 98.63 88.2992) (end 98.63 87.733515) (width 0.5) (layer B.Cu) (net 2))
 (via (at 111.21644 81.56956) (size 0.8) (drill 0.4) (layers F.Cu B.Cu) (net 2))
 (segment (start 111.258599 81.611719) (end 111.21644 81.56956) (width 0.5) (layer B.Cu) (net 2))
 (segment (start 111.258599 88.650001) (end 111.258599 81.611719) (width 0.5) (layer B.Cu) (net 2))
 (segment (start 111.21644 80.87116) (end 113.107 78.9806) (width 0.5) (layer F.Cu) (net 2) (status 20))
 (segment (start 111.21644 81.56956) (end 111.21644 80.87116) (width 0.5) (layer F.Cu) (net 2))
 (segment (start 119.545002 83.08) (end 118.93 83.08) (width 0.5) (layer F.Cu) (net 2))
 (segment (start 119.930001 83.464999) (end 119.545002 83.08) (width 0.5) (layer F.Cu) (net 2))
 (segment (start 119.930001 87.794999) (end 119.930001 83.464999) (width 0.5) (layer F.Cu) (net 2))
 (segment (start 118.93 88.795) (end 119.930001 87.794999) (width 0.5) (layer F.Cu) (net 2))
 (segment (start 98.63 78.825) (end 98.63 80.025) (width 0.4) (layer F.Cu) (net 4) (status 30))
 (segment (start 102.92 85.175) (end 105.205 85.175) (width 0.25) (layer F.Cu) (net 4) (status 20))
 (segment (start 98.63 80.885) (end 102.92 85.175) (width 0.25) (layer F.Cu) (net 4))
 (segment (start 98.63 79.135) (end 98.63 80.885) (width 0.25) (layer F.Cu) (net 4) (status 10))
 (segment (start 99.9 78.825) (end 99.9 80.025) (width 0.4) (layer F.Cu) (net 5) (status 30))
 (segment (start 102.92 83.905) (end 105.205 83.905) (width 0.25) (layer F.Cu) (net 5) (status 20))
 (segment (start 99.9 80.885) (end 102.92 83.905) (width 0.25) (layer F.Cu) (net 5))
 (segment (start 99.9 79.135) (end 99.9 80.885) (width 0.25) (layer F.Cu) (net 5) (status 10))
 (segment (start 104.67 82.635) (end 105.205 82.635) (width 0.25) (layer F.Cu) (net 6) (status 30))
 (segment (start 101.17 79.135) (end 104.67 82.635) (width 0.25) (layer F.Cu) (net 6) (status 30))
 (segment (start 118.635 84.08) (end 118.93 84.08) (width 0.25) (layer F.Cu) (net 8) (status 30))
 (segment (start 118.755 83.905) (end 118.93 84.08) (width 0.25) (layer F.Cu) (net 8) (status 30))
 (segment (start 116.904601 83.741999) (end 116.904601 81.534401) (width 0.25) (layer F.Cu) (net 8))
 (segment (start 116.7416 83.905) (end 116.904601 83.741999) (width 0.25) (layer F.Cu) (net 8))
 (segment (start 114.505 83.905) (end 116.7416 83.905) (width 0.25) (layer F.Cu) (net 8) (status 10))
 (segment (start 116.7416 83.905) (end 118.755 83.905) (width 0.25) (layer F.Cu) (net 8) (status 20))
 (segment (start 120.035399 80.006001) (end 121.2104 78.831) (width 0.25) (layer F.Cu) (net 8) (status 20))
 (segment (start 118.433001 80.006001) (end 120.035399 80.006001) (width 0.25) (layer F.Cu) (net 8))
 (segment (start 116.904601 81.534401) (end 118.433001 80.006001) (width 0.25) (layer F.Cu) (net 8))
 (segment (start 118.635 85.08) (end 118.93 85.08) (width 0.25) (layer F.Cu) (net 7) (status 30))
 (segment (start 118.835 85.175) (end 118.93 85.08) (width 0.25) (layer F.Cu) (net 7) (status 30))
 (via (at 117.7036 85.09499) (size 0.8) (drill 0.4) (layers F.Cu B.Cu) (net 7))
 (segment (start 117.7068 85.09819) (end 117.7036 85.09499) (width 0.25) (layer F.Cu) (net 7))
 (segment (start 117.7068 85.175) (end 117.7068 85.09819) (width 0.25) (layer F.Cu) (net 7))
 (segment (start 114.505 85.175) (end 117.7068 85.175) (width 0.25) (layer F.Cu) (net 7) (status 10))
 (segment (start 117.7068 85.175) (end 118.835 85.175) (width 0.25) (layer F.Cu) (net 7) (status 20))
 (via (at 118.3132 81.4698) (size 0.8) (drill 0.4) (layers F.Cu B.Cu) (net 7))
 (segment (start 117.7036 82.0794) (end 118.3132 81.4698) (width 0.25) (layer B.Cu) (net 7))
 (segment (start 117.7036 85.09499) (end 117.7036 82.0794) (width 0.25) (layer B.Cu) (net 7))
 (segment (start 122.949402 78.831) (end 123.7504 78.831) (width 0.25) (layer F.Cu) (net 7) (status 30))
 (segment (start 120.310602 81.4698) (end 122.949402 78.831) (width 0.25) (layer F.Cu) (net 7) (status 20))
 (segment (start 118.3132 81.4698) (end 120.310602 81.4698) (width 0.25) (layer F.Cu) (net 7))
 (segment (start 118.8918 86.0418) (end 118.93 86.08) (width 0.25) (layer F.Cu) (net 33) (status 30))
 (via (at 116.1796 86.0926) (size 0.8) (drill 0.4) (layers F.Cu B.Cu) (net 33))
 (segment (start 116.45221 85.81999) (end 116.1796 86.0926) (width 0.25) (layer F.Cu) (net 33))
 (segment (start 118.66999 85.81999) (end 116.45221 85.81999) (width 0.25) (layer F.Cu) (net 33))
 (segment (start 118.93 86.08) (end 118.66999 85.81999) (width 0.25) (layer F.Cu) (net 33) (status 10))
 (via (at 116.1796 82.689) (size 0.8) (drill 0.4) (layers F.Cu B.Cu) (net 33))
 (segment (start 116.1796 86.0926) (end 116.1796 82.689) (width 0.25) (layer B.Cu) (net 33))
 (segment (start 114.559 82.689) (end 114.505 82.635) (width 0.25) (layer F.Cu) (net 33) (status 30))
 (segment (start 116.1796 82.689) (end 114.559 82.689) (width 0.25) (layer F.Cu) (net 33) (status 20))
 (segment (start 118.295 87.715) (end 118.93 87.08) (width 0.25) (layer F.Cu) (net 32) (status 20))
 (segment (start 114.505 87.715) (end 118.295 87.715) (width 0.25) (layer F.Cu) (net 32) (status 10))
 (segment (start 118.510001 89.375001) (end 118.93 89.795) (width 0.25) (layer F.Cu) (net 31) (status 20))
 (segment (start 114.895001 89.375001) (end 118.510001 89.375001) (width 0.25) (layer F.Cu) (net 31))
 (segment (start 114.505 88.985) (end 114.895001 89.375001) (width 0.25) (layer F.Cu) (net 31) (status 10))
 (segment (start 115.045 90.795) (end 118.93 90.795) (width 0.25) (layer F.Cu) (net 30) (status 20))
 (segment (start 114.505 90.255) (end 115.045 90.795) (width 0.25) (layer F.Cu) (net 30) (status 10))
 (segment (start 118.66 91.525) (end 118.93 91.795) (width 0.25) (layer F.Cu) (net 29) (status 20))
 (segment (start 114.505 91.525) (end 118.66 91.525) (width 0.25) (layer F.Cu) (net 29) (status 10))
 (segment (start 114.505 92.795) (end 118.93 92.795) (width 0.25) (layer F.Cu) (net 28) (status 30))
 (segment (start 103.275 91.89) (end 101.18 91.89) (width 0.25) (layer F.Cu) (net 27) (status 20))
 (segment (start 104.18 92.795) (end 103.275 91.89) (width 0.25) (layer F.Cu) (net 27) (status 10))
 (segment (start 105.205 92.795) (end 104.18 92.795) (width 0.25) (layer F.Cu) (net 27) (status 30))
 (segment (start 104.57 90.89) (end 101.18 90.89) (width 0.25) (layer F.Cu) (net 26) (status 20))
 (segment (start 105.205 91.525) (end 104.57 90.89) (width 0.25) (layer F.Cu) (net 26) (status 10))
 (segment (start 101.545 90.255) (end 101.18 89.89) (width 0.25) (layer F.Cu) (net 25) (status 20))
 (segment (start 105.205 90.255) (end 101.545 90.255) (width 0.25) (layer F.Cu) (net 25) (status 10))
 (segment (start 101.275 88.985) (end 101.18 88.89) (width 0.25) (layer F.Cu) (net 24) (status 30))
 (segment (start 105.205 88.985) (end 101.275 88.985) (width 0.25) (layer F.Cu) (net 24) (status 30))
 (via (at 97.4362 89.874) (size 0.8) (drill 0.4) (layers F.Cu B.Cu) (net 20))
 (segment (start 97.4202 89.89) (end 97.4362 89.874) (width 0.4) (layer F.Cu) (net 20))
 (segment (start 96.08 89.89) (end 97.4202 89.89) (width 0.4) (layer F.Cu) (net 20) (status 10))
 (segment (start 96.5472 88.985) (end 92.915 88.985) (width 0.4) (layer B.Cu) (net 20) (status 20))
 (segment (start 97.4362 89.874) (end 96.5472 88.985) (width 0.4) (layer B.Cu) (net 20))
 (via (at 97.230002 92.1092) (size 0.8) (drill 0.4) (layers F.Cu B.Cu) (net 21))
 (segment (start 97.03 90.89) (end 97.230002 91.090002) (width 0.4) (layer F.Cu) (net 21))
 (segment (start 97.230002 91.090002) (end 97.230002 92.1092) (width 0.4) (layer F.Cu) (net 21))
 (segment (start 96.08 90.89) (end 97.03 90.89) (width 0.4) (layer F.Cu) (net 21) (status 10))
 (segment (start 92.9658 92.1092) (end 92.915 92.16) (width 0.4) (layer B.Cu) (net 21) (status 30))
 (segment (start 97.230002 92.1092) (end 92.9658 92.1092) (width 0.4) (layer B.Cu) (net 21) (status 20))
 (via (at 122.6076 84.667) (size 0.8) (drill 0.4) (layers F.Cu B.Cu) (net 14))
 (segment (start 123.1946 84.08) (end 122.6076 84.667) (width 0.4) (layer F.Cu) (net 14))
 (segment (start 124.03 84.08) (end 123.1946 84.08) (width 0.4) (layer F.Cu) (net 14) (status 10))
 (segment (start 123.7506 85.81) (end 126.57 85.81) (width 0.4) (layer B.Cu) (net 14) (status 20))
 (segment (start 122.6076 84.667) (end 123.7506 85.81) (width 0.4) (layer B.Cu) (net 14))
 (via (at 124.0554 81.9238) (size 0.8) (drill 0.4) (layers F.Cu B.Cu) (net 15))
 (segment (start 124.03 81.9492) (end 124.0554 81.9238) (width 0.4) (layer F.Cu) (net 15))
 (segment (start 124.03 83.08) (end 124.03 81.9492) (width 0.4) (layer F.Cu) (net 15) (status 10))
 (segment (start 125.8588 81.9238) (end 126.57 82.635) (width 0.4) (layer B.Cu) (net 15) (status 30))
 (segment (start 124.0554 81.9238) (end 125.8588 81.9238) (width 0.4) (layer B.Cu) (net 15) (status 20))
 (segment (start 126.3 86.08) (end 126.57 85.81) (width 0.4) (layer F.Cu) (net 12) (status 30))
 (segment (start 124.03 86.08) (end 126.3 86.08) (width 0.4) (layer F.Cu) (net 12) (status 30))
 (segment (start 124.03 85.08) (end 124.426799 85.08) (width 0.4) (layer F.Cu) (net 13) (status 30))
 (segment (start 126.57 82.936799) (end 126.57 82.635) (width 0.4) (layer F.Cu) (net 13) (status 30))
 (segment (start 124.426799 85.08) (end 126.57 82.936799) (width 0.4) (layer F.Cu) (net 13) (status 30)))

